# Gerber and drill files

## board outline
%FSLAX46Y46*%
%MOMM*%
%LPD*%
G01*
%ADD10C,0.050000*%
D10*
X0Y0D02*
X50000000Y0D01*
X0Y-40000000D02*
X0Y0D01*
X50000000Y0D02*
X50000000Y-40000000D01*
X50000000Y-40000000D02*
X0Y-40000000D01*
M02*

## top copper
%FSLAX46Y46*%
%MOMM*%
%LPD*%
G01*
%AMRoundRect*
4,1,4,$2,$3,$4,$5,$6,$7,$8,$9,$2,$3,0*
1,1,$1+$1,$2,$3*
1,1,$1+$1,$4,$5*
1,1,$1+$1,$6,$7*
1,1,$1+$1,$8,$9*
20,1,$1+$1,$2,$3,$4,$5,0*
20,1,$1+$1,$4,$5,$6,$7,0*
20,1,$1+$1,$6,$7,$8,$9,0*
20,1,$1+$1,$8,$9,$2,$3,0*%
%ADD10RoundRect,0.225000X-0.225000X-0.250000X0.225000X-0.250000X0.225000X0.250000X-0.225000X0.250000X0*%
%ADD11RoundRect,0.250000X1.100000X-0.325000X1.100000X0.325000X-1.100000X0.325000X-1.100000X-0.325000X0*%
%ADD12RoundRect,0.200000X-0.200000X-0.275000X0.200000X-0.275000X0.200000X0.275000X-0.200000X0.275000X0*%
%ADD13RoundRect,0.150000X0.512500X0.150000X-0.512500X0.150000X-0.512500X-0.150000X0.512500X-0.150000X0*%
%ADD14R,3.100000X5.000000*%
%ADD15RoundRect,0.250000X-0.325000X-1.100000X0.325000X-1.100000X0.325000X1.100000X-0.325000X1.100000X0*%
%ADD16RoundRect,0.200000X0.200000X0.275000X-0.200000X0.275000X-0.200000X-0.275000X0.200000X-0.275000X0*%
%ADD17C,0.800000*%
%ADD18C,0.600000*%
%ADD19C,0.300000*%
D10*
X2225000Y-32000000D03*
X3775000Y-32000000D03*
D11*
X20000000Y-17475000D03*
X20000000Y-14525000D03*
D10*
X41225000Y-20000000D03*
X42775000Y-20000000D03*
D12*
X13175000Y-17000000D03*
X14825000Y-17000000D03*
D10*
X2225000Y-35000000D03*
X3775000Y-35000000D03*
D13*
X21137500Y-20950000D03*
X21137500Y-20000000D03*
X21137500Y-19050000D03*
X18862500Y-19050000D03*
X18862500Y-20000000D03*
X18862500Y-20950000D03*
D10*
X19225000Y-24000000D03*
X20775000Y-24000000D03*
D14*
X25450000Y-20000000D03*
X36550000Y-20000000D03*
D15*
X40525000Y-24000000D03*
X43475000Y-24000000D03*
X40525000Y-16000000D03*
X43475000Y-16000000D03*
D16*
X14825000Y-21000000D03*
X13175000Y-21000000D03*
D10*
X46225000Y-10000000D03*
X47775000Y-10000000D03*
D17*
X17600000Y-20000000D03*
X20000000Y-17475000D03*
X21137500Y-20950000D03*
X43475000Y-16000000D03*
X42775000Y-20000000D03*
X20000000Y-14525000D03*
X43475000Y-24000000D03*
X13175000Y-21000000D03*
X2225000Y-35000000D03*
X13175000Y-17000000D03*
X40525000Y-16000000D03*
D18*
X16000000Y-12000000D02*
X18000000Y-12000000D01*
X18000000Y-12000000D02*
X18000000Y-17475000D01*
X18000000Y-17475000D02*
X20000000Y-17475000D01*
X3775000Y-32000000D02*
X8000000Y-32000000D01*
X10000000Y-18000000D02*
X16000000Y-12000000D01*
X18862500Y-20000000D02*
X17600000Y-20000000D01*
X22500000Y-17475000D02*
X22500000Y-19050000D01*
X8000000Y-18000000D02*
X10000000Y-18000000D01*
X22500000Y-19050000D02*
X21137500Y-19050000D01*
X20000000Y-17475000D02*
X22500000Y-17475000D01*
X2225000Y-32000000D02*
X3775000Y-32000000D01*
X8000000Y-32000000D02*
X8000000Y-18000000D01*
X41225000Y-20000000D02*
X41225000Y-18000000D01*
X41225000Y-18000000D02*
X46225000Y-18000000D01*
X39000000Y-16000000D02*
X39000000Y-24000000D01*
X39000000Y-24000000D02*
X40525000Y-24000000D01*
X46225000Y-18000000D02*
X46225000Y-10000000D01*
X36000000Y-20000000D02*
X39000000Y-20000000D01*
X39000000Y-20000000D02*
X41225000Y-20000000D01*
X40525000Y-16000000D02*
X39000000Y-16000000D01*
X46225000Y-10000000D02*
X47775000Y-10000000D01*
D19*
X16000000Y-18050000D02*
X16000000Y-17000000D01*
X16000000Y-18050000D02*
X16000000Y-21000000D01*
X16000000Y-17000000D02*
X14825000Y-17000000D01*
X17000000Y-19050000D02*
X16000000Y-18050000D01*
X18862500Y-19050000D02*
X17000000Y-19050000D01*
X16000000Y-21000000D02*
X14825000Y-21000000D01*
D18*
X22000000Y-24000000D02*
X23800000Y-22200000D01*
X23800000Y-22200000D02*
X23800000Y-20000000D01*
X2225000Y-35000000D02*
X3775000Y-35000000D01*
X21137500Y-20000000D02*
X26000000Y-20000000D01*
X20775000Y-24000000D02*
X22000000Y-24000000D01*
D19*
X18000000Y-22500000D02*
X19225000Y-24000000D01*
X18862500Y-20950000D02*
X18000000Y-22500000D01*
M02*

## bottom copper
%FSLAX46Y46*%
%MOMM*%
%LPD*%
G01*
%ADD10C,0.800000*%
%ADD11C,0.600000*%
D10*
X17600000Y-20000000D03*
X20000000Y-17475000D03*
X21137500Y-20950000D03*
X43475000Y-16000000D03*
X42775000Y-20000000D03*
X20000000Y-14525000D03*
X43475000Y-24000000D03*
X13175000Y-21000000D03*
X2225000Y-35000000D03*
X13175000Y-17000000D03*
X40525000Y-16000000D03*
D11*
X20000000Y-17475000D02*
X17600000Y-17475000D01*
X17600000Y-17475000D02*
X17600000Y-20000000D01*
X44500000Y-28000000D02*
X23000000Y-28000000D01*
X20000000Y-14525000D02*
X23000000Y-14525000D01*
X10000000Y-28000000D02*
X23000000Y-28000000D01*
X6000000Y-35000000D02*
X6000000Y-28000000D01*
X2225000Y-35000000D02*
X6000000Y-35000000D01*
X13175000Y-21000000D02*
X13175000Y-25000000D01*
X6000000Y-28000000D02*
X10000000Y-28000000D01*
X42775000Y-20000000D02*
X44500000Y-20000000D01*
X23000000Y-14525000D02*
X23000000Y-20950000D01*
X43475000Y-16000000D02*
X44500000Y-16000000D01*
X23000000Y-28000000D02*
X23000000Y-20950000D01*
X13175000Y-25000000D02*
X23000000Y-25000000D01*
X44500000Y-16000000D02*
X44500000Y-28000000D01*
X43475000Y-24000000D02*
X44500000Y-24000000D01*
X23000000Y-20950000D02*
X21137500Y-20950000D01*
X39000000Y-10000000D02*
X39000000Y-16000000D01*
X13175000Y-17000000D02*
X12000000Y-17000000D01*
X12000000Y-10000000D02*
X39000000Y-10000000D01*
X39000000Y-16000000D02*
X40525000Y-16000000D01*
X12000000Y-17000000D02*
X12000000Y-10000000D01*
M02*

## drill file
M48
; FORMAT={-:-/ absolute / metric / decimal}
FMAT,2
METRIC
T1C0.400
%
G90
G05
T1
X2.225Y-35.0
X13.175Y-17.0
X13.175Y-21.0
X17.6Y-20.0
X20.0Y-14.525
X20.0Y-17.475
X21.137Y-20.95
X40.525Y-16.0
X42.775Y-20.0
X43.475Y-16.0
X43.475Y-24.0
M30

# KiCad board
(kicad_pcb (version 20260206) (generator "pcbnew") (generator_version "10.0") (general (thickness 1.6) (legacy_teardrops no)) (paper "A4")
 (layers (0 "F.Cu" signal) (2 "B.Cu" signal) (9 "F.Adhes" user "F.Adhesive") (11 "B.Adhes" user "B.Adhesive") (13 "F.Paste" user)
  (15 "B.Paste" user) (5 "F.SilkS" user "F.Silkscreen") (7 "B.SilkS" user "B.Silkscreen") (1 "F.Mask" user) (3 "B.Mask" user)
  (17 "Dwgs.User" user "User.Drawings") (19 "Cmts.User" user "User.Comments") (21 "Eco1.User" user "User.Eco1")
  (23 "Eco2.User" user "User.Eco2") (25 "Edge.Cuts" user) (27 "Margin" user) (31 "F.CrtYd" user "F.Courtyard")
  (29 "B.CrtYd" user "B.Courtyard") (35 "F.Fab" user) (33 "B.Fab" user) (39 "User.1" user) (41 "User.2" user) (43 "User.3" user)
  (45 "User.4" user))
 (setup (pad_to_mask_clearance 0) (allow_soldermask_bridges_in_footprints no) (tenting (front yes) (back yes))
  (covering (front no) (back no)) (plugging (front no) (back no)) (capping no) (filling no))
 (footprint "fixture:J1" (layer "F.Cu") (at 3 32)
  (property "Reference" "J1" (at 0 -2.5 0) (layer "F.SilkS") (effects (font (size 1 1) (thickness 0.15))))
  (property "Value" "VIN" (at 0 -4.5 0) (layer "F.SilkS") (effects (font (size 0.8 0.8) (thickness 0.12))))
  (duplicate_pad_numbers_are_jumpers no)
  (pad "1" smd roundrect (at -0.775 0) (size 0.9 0.95) (layers "F.Cu" "F.Mask" "F.Paste") (roundrect_rratio 0.25) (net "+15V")
   (thermal_bridge_angle 45))
  (pad "2" smd roundrect (at 0.775 0) (size 0.9 0.95) (layers "F.Cu" "F.Mask" "F.Paste") (roundrect_rratio 0.25) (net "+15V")
   (thermal_bridge_angle 45)))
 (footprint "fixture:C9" (layer "F.Cu") (at 20 16 90)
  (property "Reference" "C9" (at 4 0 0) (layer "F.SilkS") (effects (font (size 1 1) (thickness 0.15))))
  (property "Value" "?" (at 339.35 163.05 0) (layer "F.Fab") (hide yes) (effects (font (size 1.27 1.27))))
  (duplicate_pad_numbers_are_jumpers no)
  (pad "1" smd roundrect (at -1.475 0 90) (size 1.15 2.7) (layers "F.Cu" "F.Mask" "F.Paste") (roundrect_rratio 0.217391) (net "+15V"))
  (pad "2" smd roundrect (at 1.475 0 90) (size 1.15 2.7) (layers "F.Cu" "F.Mask" "F.Paste") (roundrect_rratio 0.217391) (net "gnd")))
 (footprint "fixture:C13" (layer "F.Cu") (at 42 20)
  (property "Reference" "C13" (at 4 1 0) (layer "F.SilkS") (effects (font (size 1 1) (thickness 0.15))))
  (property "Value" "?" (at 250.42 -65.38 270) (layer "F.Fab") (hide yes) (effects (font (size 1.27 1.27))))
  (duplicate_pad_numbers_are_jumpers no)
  (pad "1" smd roundrect (at -0.775 0) (size 0.9 0.95) (layers "F.Cu" "F.Mask" "F.Paste") (roundrect_rratio 0.25) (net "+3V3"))
  (pad "2" smd roundrect (at 0.775 0) (size 0.9 0.95) (layers "F.Cu" "F.Mask" "F.Paste") (roundrect_rratio 0.25) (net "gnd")))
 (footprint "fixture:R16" (layer "F.Cu") (at 14 17)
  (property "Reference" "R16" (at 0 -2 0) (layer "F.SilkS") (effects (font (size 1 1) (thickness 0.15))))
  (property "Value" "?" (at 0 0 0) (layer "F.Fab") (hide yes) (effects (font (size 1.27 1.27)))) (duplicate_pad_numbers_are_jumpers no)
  (pad "1" smd roundrect (at -0.825 0) (size 0.8 0.95) (layers "F.Cu" "F.Mask" "F.Paste") (roundrect_rratio 0.25) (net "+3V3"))
  (pad "2" smd roundrect (at 0.825 0) (size 0.8 0.95) (layers "F.Cu" "F.Mask" "F.Paste") (roundrect_rratio 0.25) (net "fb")))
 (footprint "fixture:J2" (layer "F.Cu") (at 3 35)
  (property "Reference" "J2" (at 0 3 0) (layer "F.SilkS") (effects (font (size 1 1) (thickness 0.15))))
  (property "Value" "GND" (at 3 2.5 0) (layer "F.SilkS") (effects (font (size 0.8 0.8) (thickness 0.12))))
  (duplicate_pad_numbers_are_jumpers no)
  (pad "1" smd roundrect (at -0.775 0) (size 0.9 0.95) (layers "F.Cu" "F.Mask" "F.Paste") (roundrect_rratio 0.25) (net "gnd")
   (thermal_bridge_angle 45))
  (pad "2" smd roundrect (at 0.775 0) (size 0.9 0.95) (layers "F.Cu" "F.Mask" "F.Paste") (roundrect_rratio 0.25) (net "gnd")
   (thermal_bridge_angle 45)))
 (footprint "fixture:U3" (layer "F.Cu") (at 20 20 180)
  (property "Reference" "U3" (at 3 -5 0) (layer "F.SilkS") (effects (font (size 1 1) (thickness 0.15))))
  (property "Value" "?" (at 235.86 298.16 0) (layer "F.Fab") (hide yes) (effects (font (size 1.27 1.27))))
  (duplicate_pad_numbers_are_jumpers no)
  (pad "1" smd roundrect (at -1.1375 -0.95 180) (size 1.325 0.6) (layers "F.Cu" "F.Mask" "F.Paste") (roundrect_rratio 0.25) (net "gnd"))
  (pad "2" smd roundrect (at -1.1375 0 180) (size 1.325 0.6) (layers "F.Cu" "F.Mask" "F.Paste") (roundrect_rratio 0.25) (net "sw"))
  (pad "3" smd roundrect (at -1.1375 0.95 180) (size 1.325 0.6) (layers "F.Cu" "F.Mask" "F.Paste") (roundrect_rratio 0.25) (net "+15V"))
  (pad "4" smd roundrect (at 1.1375 0.95 180) (size 1.325 0.6) (layers "F.Cu" "F.Mask" "F.Paste") (roundrect_rratio 0.25) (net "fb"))
  (pad "5" smd roundrect (at 1.1375 0 180) (size 1.325 0.6) (layers "F.Cu" "F.Mask" "F.Paste") (roundrect_rratio 0.25) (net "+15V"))
  (pad "6" smd roundrect (at 1.1375 -0.95 180) (size 1.325 0.6) (layers "F.Cu" "F.Mask" "F.Paste") (roundrect_rratio 0.25) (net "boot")))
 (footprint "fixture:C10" (layer "F.Cu") (at 20 24)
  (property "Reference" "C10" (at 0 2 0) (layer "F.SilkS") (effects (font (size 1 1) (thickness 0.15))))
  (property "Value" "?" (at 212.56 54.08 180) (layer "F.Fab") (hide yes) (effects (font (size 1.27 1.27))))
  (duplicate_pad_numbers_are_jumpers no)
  (pad "1" smd roundrect (at -0.775 0) (size 0.9 0.95) (layers "F.Cu" "F.Mask" "F.Paste") (roundrect_rratio 0.25) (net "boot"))
  (pad "2" smd roundrect (at 0.775 0) (size 0.9 0.95) (layers "F.Cu" "F.Mask" "F.Paste") (roundrect_rratio 0.25) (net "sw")))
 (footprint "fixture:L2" (layer "F.Cu") (at 31 20)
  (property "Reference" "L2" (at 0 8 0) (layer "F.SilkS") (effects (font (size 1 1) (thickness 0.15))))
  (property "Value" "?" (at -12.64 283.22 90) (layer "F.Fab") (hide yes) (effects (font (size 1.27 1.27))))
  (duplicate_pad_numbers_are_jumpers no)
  (pad "1" smd rect (at -5.55 0) (size 3.1 5) (layers "F.Cu" "F.Mask" "F.Paste") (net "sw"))
  (pad "2" smd rect (at 5.55 0) (size 3.1 5) (layers "F.Cu" "F.Mask" "F.Paste") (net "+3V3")))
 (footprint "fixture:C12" (layer "F.Cu") (at 42 24)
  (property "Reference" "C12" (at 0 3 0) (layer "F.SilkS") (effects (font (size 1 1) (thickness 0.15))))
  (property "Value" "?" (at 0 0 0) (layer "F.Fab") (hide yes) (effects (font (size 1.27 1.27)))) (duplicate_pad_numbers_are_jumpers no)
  (pad "1" smd roundrect (at -1.475 0) (size 1.15 2.7) (layers "F.Cu" "F.Mask" "F.Paste") (roundrect_rratio 0.217391) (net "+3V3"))
  (pad "2" smd roundrect (at 1.475 0) (size 1.15 2.7) (layers "F.Cu" "F.Mask" "F.Paste") (roundrect_rratio 0.217391) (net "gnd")))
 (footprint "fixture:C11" (layer "F.Cu") (at 42 16)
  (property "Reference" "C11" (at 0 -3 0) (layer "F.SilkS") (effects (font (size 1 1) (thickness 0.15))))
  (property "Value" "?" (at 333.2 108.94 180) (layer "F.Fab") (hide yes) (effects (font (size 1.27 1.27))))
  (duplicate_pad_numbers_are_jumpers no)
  (pad "1" smd roundrect (at -1.475 0) (size 1.15 2.7) (layers "F.Cu" "F.Mask" "F.Paste") (roundrect_rratio 0.217391) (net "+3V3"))
  (pad "2" smd roundrect (at 1.475 0) (size 1.15 2.7) (layers "F.Cu" "F.Mask" "F.Paste") (roundrect_rratio 0.217391) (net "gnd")))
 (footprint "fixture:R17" (layer "F.Cu") (at 14 21 180)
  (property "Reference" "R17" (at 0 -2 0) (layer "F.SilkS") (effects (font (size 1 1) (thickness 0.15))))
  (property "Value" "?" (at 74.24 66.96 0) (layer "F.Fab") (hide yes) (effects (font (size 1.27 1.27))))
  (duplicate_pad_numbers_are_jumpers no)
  (pad "1" smd roundrect (at -0.825 0 180) (size 0.8 0.95) (layers "F.Cu" "F.Mask" "F.Paste") (roundrect_rratio 0.25) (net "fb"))
  (pad "2" smd roundrect (at 0.825 0 180) (size 0.8 0.95) (layers "F.Cu" "F.Mask" "F.Paste") (roundrect_rratio 0.25) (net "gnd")))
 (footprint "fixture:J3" (layer "F.Cu") (at 47 10)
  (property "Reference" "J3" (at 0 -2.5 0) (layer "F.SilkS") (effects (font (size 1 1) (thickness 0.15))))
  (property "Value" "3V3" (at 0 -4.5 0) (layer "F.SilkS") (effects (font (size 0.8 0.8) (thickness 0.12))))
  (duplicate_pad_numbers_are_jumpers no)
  (pad "1" smd roundrect (at -0.775 0) (size 0.9 0.95) (layers "F.Cu" "F.Mask" "F.Paste") (roundrect_rratio 0.25) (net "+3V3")
   (thermal_bridge_angle 45))
  (pad "2" smd roundrect (at 0.775 0) (size 0.9 0.95) (layers "F.Cu" "F.Mask" "F.Paste") (roundrect_rratio 0.25) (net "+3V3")
   (thermal_bridge_angle 45)))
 (gr_line (start 0 0) (end 50 0) (stroke (width 0.05) (type default)) (layer "Edge.Cuts"))
 (gr_line (start 0 40) (end 0 0) (stroke (width 0.05) (type default)) (layer "Edge.Cuts"))
 (gr_line (start 50 0) (end 50 40) (stroke (width 0.05) (type default)) (layer "Edge.Cuts"))
 (gr_line (start 50 40) (end 0 40) (stroke (width 0.05) (type default)) (layer "Edge.Cuts"))
 (segment (start 16 12) (end 18 12) (width 0.6) (layer "F.Cu") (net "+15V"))
 (segment (start 18 12) (end 18 17.475) (width 0.6) (layer "F.Cu") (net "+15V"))
 (segment (start 18 17.475) (end 20 17.475) (width 0.6) (layer "F.Cu") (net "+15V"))
 (segment (start 3.775 32) (end 8 32) (width 0.6) (layer "F.Cu") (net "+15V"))
 (segment (start 10 18) (end 16 12) (width 0.6) (layer "F.Cu") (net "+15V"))
 (segment (start 18.8625 20) (end 17.6 20) (width 0.6) (layer "F.Cu") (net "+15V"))
 (segment (start 22.5 17.475) (end 22.5 19.05) (width 0.6) (layer "F.Cu") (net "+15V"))
 (segment (start 8 18) (end 10 18) (width 0.6) (layer "F.Cu") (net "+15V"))
 (segment (start 22.5 19.05) (end 21.1375 19.05) (width 0.6) (layer "F.Cu") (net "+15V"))
 (segment (start 20 17.475) (end 22.5 17.475) (width 0.6) (layer "F.Cu") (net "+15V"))
 (segment (start 2.225 32) (end 3.775 32) (width 0.6) (layer "F.Cu") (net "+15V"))
 (segment (start 8 32) (end 8 18) (width 0.6) (layer "F.Cu") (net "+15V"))
 (via (at 17.6 20) (size 0.8) (drill 0.4) (layers "F.Cu" "B.Cu") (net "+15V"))
 (via (at 20 17.475) (size 0.8) (drill 0.4) (layers "F.Cu" "B.Cu") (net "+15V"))
 (segment (start 20 17.475) (end 17.6 17.475) (width 0.6) (layer "B.Cu") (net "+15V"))
 (segment (start 17.6 17.475) (end 17.6 20) (width 0.6) (layer "B.Cu") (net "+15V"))
 (via (at 21.1375 20.95) (size 0.8) (drill 0.4) (layers "F.Cu" "B.Cu") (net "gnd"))
 (via (at 43.475 16) (size 0.8) (drill 0.4) (layers "F.Cu" "B.Cu") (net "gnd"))
 (via (at 42.775 20) (size 0.8) (drill 0.4) (layers "F.Cu" "B.Cu") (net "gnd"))
 (via (at 20 14.525) (size 0.8) (drill 0.4) (layers "F.Cu" "B.Cu") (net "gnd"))
 (via (at 43.475 24) (size 0.8) (drill 0.4) (layers "F.Cu" "B.Cu") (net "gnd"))
 (via (at 13.175 21) (size 0.8) (drill 0.4) (layers "F.Cu" "B.Cu") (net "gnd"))
 (via (at 2.225 35) (size 0.8) (drill 0.4) (layers "F.Cu" "B.Cu") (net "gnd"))
 (segment (start 44.5 28) (end 23 28) (width 0.6) (layer "B.Cu") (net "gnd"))
 (segment (start 20 14.525) (end 23 14.525) (width 0.6) (layer "B.Cu") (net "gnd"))
 (segment (start 10 28) (end 23 28) (width 0.6) (layer "B.Cu") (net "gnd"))
 (segment (start 6 35) (end 6 28) (width 0.6) (layer "B.Cu") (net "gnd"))
 (segment (start 2.225 35) (end 6 35) (width 0.6) (layer "B.Cu") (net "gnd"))
 (segment (start 13.175 21) (end 13.175 25) (width 0.6) (layer "B.Cu") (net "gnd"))
 (segment (start 6 28) (end 10 28) (width 0.6) (layer "B.Cu") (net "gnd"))
 (segment (start 42.775 20) (end 44.5 20) (width 0.6) (layer "B.Cu") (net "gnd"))
 (segment (start 23 14.525) (end 23 20.95) (width 0.6) (layer "B.Cu") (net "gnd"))
 (segment (start 43.475 16) (end 44.5 16) (width 0.6) (layer "B.Cu") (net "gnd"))
 (segment (start 23 28) (end 23 20.95) (width 0.6) (layer "B.Cu") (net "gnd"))
 (segment (start 13.175 25) (end 23 25) (width 0.6) (layer "B.Cu") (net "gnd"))
 (segment (start 44.5 16) (end 44.5 28) (width 0.6) (layer "B.Cu") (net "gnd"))
 (segment (start 43.475 24) (end 44.5 24) (width 0.6) (layer "B.Cu") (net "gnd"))
 (segment (start 23 20.95) (end 21.1375 20.95) (width 0.6) (layer "B.Cu") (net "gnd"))
 (segment (start 41.225 20) (end 41.225 18) (width 0.6) (layer "F.Cu") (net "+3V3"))
 (segment (start 41.225 18) (end 46.225 18) (width 0.6) (layer "F.Cu") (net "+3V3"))
 (segment (start 39 16) (end 39 24) (width 0.6) (layer "F.Cu") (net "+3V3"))
 (segment (start 39 24) (end 40.525 24) (width 0.6) (layer "F.Cu") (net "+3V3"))
 (segment (start 46.225 18) (end 46.225 10) (width 0.6) (layer "F.Cu") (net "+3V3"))
 (segment (start 36 20) (end 39 20) (width 0.6) (layer "F.Cu") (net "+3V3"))
 (segment (start 39 20) (end 41.225 20) (width 0.6) (layer "F.Cu") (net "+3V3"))
 (segment (start 40.525 16) (end 39 16) (width 0.6) (layer "F.Cu") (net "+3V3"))
 (segment (start 46.225 10) (end 47.775 10) (width 0.6) (layer "F.Cu") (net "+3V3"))
 (via (at 13.175 17) (size 0.8) (drill 0.4) (layers "F.Cu" "B.Cu") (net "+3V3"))
 (via (at 40.525 16) (size 0.8) (drill 0.4) (layers "F.Cu" "B.Cu") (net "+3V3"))
 (segment (start 39 10) (end 39 16) (width 0.6) (layer "B.Cu") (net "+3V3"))
 (segment (start 13.175 17) (end 12 17) (width 0.6) (layer "B.Cu") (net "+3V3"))
 (segment (start 12 10) (end 39 10) (width 0.6) (layer "B.Cu") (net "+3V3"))
 (segment (start 39 16) (end 40.525 16) (width 0.6) (layer "B.Cu") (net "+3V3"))
 (segment (start 12 17) (end 12 10) (width 0.6) (layer "B.Cu") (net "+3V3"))
 (segment (start 16 18.05) (end 16 17) (width 0.3) (layer "F.Cu") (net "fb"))
 (segment (start 16 18.05) (end 16 21) (width 0.3) (layer "F.Cu") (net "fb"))
 (segment (start 16 17) (end 14.825 17) (width 0.3) (layer "F.Cu") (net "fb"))
 (segment (start 17 19.05) (end 16 18.05) (width 0.3) (layer "F.Cu") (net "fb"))
 (segment (start 18.8625 19.05) (end 17 19.05) (width 0.3) (layer "F.Cu") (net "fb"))
 (segment (start 16 21) (end 14.825 21) (width 0.3) (layer "F.Cu") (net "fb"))
 (segment (start 22 24) (end 23.8 22.2) (width 0.6) (layer "F.Cu") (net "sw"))
 (segment (start 23.8 22.2) (end 23.8 20) (width 0.6) (layer "F.Cu") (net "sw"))
 (segment (start 2.225 35) (end 3.775 35) (width 0.6) (layer "F.Cu") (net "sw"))
 (segment (start 21.1375 20) (end 26 20) (width 0.6) (layer "F.Cu") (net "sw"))
 (segment (start 20.775 24) (end 22 24) (width 0.6) (layer "F.Cu") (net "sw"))
 (segment (start 18 22.5) (end 19.225 24) (width 0.3) (layer "F.Cu") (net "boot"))
 (segment (start 18.8625 20.95) (end 18 22.5) (width 0.3) (layer "F.Cu") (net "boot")))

